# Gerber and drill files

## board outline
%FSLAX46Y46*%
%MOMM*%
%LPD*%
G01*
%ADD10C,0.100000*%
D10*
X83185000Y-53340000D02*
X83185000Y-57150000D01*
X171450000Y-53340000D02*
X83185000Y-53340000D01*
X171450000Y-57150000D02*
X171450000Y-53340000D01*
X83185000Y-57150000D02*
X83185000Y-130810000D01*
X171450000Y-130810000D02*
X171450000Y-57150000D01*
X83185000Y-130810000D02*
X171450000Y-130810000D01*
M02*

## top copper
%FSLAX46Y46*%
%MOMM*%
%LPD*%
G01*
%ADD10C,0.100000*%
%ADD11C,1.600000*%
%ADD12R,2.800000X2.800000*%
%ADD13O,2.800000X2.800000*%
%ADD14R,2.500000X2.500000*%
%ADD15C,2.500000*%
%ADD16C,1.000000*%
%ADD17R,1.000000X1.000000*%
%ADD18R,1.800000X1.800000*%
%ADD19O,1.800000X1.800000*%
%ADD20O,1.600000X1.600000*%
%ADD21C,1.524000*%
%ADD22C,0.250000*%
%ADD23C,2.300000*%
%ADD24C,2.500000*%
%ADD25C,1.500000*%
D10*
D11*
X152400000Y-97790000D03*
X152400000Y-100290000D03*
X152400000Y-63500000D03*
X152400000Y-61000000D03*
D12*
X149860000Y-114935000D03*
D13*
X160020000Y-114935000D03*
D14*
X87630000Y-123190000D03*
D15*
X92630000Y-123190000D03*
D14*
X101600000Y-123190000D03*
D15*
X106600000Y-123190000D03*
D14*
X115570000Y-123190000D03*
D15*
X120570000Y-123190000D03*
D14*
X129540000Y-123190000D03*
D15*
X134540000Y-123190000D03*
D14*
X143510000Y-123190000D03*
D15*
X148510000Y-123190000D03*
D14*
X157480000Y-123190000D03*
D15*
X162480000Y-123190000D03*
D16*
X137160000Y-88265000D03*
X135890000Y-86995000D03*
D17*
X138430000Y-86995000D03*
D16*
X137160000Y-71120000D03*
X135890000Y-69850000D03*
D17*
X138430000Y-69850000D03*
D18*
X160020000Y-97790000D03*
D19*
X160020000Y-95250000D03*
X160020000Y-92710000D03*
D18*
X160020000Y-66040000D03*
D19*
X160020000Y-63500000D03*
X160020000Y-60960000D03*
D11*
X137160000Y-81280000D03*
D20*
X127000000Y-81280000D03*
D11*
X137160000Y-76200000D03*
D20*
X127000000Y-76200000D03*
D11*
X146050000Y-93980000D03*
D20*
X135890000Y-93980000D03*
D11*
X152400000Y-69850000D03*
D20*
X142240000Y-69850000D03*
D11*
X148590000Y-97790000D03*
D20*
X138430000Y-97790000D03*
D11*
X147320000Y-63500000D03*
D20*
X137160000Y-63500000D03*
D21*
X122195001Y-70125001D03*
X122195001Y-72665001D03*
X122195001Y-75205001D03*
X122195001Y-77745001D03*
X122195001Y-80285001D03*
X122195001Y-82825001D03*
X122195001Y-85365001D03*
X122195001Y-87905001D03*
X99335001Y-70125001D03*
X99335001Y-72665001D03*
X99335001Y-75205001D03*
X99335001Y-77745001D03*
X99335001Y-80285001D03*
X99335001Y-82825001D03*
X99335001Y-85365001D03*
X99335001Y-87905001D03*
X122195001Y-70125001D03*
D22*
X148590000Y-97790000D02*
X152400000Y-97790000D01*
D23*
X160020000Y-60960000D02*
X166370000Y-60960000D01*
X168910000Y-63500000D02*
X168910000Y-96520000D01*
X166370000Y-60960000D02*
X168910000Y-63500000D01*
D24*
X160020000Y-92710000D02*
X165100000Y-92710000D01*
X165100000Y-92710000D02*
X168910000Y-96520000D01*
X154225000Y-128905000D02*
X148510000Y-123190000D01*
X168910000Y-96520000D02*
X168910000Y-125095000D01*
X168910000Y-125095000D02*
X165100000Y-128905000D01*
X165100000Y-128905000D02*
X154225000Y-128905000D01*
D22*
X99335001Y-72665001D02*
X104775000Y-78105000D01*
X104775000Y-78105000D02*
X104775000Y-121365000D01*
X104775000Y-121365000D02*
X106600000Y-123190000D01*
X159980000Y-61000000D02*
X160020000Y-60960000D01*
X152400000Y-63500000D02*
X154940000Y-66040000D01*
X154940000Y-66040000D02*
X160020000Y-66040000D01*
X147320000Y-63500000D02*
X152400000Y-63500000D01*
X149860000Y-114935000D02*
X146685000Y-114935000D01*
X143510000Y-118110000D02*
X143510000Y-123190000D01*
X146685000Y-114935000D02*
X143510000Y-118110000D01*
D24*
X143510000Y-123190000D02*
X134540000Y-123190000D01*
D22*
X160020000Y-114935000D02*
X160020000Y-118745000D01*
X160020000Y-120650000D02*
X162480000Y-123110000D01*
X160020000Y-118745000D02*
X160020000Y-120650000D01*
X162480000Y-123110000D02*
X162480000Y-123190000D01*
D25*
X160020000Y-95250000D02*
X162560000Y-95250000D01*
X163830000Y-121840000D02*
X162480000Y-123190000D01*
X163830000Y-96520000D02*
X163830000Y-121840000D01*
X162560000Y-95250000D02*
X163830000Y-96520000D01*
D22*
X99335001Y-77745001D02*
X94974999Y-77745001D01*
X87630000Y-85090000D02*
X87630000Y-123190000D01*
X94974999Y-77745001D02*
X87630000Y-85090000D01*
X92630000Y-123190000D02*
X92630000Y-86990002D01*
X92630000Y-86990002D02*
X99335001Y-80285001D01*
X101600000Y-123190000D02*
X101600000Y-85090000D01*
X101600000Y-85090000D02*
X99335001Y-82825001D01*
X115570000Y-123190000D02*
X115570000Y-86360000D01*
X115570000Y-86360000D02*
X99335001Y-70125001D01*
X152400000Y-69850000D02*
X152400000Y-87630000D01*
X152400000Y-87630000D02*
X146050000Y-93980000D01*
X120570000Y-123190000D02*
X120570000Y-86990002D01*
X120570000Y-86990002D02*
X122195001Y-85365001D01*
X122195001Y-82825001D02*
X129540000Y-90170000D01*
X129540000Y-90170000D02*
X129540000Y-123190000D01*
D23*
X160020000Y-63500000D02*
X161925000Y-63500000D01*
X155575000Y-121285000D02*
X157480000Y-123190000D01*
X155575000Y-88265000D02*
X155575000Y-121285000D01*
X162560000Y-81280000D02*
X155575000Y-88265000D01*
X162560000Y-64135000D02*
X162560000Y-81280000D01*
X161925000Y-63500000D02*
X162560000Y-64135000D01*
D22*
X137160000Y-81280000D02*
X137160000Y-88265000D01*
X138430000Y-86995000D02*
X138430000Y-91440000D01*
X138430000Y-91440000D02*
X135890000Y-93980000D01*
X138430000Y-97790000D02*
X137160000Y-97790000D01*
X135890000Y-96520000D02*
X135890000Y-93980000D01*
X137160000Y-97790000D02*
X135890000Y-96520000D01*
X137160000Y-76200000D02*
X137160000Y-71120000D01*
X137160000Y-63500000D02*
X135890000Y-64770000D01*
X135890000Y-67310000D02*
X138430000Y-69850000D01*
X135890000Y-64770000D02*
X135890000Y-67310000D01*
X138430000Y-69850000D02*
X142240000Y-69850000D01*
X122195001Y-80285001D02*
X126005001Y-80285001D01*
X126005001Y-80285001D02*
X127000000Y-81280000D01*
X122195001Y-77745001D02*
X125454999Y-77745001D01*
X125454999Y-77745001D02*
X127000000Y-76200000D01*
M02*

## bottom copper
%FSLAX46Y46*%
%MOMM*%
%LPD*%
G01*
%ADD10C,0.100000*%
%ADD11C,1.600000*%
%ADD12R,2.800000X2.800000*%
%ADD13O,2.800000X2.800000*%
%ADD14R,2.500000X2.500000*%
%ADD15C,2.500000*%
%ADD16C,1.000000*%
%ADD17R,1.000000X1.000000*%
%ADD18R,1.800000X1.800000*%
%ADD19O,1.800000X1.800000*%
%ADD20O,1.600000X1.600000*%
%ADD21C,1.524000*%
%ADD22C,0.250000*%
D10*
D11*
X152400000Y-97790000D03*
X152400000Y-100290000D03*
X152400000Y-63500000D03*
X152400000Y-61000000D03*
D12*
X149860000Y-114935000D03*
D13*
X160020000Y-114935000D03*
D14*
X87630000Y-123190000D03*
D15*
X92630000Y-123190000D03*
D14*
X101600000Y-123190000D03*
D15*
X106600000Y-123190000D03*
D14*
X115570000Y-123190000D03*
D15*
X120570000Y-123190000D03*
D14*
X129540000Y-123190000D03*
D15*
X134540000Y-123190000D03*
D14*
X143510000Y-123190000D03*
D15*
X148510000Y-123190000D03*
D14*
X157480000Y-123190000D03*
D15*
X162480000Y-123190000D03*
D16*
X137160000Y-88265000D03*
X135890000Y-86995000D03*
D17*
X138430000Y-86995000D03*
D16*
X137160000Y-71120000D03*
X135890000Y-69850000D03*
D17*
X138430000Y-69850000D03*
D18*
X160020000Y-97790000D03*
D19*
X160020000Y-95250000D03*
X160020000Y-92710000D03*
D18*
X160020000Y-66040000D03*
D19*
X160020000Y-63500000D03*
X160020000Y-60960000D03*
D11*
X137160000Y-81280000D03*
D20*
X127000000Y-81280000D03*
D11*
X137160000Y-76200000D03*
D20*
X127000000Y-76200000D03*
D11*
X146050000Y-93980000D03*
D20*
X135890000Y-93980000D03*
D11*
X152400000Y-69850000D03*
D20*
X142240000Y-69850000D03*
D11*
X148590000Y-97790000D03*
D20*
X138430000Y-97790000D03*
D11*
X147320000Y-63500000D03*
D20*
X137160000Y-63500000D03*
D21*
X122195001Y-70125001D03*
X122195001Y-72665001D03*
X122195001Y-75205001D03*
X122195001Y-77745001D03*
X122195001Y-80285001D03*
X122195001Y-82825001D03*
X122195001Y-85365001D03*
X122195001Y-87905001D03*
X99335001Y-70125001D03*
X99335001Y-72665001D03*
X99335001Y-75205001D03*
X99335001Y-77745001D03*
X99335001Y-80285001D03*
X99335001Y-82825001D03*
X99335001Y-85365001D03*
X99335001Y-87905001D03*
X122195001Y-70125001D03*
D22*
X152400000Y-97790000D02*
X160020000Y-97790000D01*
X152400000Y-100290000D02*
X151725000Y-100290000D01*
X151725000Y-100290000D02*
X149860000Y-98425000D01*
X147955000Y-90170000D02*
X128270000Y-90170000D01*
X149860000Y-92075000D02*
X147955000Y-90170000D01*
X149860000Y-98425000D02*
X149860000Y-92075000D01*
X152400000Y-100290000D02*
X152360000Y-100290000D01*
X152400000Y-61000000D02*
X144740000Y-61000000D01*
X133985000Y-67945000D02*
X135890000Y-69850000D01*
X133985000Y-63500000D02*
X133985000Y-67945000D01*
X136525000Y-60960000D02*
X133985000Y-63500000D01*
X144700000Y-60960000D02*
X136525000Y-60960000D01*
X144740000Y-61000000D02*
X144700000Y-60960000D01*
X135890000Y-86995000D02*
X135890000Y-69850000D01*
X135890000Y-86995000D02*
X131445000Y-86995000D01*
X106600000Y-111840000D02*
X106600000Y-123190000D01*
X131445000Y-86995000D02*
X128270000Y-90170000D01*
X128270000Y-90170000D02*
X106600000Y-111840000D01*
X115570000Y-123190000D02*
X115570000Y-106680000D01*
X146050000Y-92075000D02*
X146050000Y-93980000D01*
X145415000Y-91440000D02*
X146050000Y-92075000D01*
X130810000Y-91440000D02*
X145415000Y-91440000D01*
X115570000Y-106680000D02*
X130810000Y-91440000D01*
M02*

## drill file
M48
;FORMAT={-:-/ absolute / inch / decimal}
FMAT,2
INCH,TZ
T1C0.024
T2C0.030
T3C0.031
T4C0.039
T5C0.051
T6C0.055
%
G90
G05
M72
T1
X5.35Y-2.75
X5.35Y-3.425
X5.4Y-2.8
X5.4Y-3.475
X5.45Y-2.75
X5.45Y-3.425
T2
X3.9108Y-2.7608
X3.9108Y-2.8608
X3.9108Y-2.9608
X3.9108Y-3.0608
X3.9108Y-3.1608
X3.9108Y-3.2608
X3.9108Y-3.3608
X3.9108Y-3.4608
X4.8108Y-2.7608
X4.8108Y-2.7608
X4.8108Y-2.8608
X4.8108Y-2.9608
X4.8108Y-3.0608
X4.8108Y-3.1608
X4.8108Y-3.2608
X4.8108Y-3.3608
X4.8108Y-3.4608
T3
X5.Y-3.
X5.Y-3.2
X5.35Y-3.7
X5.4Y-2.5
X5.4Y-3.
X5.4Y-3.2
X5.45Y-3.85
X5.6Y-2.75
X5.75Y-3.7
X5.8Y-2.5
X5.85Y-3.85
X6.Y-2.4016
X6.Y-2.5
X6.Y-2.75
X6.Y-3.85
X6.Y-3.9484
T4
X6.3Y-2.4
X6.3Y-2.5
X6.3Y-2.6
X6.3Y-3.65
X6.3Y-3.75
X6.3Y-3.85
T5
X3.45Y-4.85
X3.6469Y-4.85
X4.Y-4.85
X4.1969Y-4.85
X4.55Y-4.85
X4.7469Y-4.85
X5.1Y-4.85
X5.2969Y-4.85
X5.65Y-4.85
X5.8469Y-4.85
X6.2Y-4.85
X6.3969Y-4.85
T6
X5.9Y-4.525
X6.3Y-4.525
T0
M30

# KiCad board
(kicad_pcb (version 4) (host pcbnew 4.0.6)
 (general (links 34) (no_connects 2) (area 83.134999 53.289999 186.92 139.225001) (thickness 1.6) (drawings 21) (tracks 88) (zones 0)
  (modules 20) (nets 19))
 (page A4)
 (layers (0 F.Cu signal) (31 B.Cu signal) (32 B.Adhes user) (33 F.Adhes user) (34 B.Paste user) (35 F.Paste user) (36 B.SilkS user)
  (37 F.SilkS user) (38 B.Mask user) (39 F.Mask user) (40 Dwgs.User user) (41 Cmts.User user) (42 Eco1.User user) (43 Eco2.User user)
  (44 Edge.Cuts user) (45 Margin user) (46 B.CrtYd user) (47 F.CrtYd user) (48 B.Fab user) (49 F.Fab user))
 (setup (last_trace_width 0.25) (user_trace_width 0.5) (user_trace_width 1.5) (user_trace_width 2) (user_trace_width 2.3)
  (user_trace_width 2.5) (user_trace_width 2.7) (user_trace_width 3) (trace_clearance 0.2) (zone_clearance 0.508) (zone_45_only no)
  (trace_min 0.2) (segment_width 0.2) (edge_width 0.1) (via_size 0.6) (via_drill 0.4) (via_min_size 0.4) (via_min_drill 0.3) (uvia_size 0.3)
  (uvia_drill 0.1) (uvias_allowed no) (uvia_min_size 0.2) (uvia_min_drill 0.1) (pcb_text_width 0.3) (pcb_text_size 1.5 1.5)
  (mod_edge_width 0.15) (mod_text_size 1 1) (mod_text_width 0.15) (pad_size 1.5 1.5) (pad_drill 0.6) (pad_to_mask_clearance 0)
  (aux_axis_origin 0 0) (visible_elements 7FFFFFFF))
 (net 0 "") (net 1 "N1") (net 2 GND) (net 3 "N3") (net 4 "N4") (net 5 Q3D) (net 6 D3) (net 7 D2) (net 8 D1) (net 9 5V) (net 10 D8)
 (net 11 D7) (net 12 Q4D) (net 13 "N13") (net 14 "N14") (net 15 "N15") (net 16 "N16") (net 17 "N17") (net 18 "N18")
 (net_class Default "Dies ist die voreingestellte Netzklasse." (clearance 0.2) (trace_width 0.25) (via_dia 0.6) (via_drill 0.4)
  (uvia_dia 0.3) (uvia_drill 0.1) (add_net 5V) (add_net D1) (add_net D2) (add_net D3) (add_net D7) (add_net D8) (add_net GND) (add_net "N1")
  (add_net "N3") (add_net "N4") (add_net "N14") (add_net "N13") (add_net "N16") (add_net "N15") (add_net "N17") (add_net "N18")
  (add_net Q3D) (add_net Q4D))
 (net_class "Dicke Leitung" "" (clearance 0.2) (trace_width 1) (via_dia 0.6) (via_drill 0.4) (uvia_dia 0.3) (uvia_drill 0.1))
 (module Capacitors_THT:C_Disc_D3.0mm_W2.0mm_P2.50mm (layer F.Cu) (at 152.4 97.79 270)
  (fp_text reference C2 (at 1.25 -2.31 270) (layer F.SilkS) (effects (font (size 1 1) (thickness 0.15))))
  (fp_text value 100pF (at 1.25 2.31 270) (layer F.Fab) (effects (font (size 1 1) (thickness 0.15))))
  (pad 1 thru_hole circle (at 0 0 270) (size 1.6 1.6) (drill 0.8) (layers *.Cu *.Mask) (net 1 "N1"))
  (pad 2 thru_hole circle (at 2.5 0 270) (size 1.6 1.6) (drill 0.8) (layers *.Cu *.Mask) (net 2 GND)))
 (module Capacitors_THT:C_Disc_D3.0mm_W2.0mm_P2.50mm (layer F.Cu) (at 152.4 63.5 90)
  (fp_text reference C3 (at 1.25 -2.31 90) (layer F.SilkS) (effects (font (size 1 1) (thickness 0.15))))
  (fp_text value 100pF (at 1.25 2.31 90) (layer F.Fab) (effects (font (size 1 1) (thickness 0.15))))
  (pad 1 thru_hole circle (at 0 0 90) (size 1.6 1.6) (drill 0.8) (layers *.Cu *.Mask) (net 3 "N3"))
  (pad 2 thru_hole circle (at 2.5 0 90) (size 1.6 1.6) (drill 0.8) (layers *.Cu *.Mask) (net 2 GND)))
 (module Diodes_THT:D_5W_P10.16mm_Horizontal (layer F.Cu) (at 149.86 114.935)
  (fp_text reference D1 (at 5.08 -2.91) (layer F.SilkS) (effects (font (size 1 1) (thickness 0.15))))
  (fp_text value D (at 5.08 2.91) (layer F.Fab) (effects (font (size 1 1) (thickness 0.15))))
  (pad 1 thru_hole rect (at 0 0) (size 2.8 2.8) (drill 1.4) (layers *.Cu *.Mask) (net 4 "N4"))
  (pad 2 thru_hole oval (at 10.16 0) (size 2.8 2.8) (drill 1.4) (layers *.Cu *.Mask) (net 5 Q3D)))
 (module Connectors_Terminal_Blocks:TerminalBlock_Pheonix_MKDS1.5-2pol (layer F.Cu) (at 87.63 123.19)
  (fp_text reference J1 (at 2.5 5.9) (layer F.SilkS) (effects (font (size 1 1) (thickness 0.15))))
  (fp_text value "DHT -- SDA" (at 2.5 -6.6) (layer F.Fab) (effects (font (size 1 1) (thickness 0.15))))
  (pad 1 thru_hole rect (at 0 0) (size 2.5 2.5) (drill 1.3) (layers *.Cu *.Mask) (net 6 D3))
  (pad 2 thru_hole circle (at 5 0) (size 2.5 2.5) (drill 1.3) (layers *.Cu *.Mask) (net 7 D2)))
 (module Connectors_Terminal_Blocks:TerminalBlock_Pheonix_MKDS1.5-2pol (layer F.Cu) (at 101.6 123.19)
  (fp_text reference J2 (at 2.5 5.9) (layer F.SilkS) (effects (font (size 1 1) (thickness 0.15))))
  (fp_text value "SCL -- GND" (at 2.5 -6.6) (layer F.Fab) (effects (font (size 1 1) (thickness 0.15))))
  (pad 1 thru_hole rect (at 0 0) (size 2.5 2.5) (drill 1.3) (layers *.Cu *.Mask) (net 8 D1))
  (pad 2 thru_hole circle (at 5 0) (size 2.5 2.5) (drill 1.3) (layers *.Cu *.Mask) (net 2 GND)))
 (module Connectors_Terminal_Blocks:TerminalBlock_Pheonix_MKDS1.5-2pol (layer F.Cu) (at 115.57 123.19)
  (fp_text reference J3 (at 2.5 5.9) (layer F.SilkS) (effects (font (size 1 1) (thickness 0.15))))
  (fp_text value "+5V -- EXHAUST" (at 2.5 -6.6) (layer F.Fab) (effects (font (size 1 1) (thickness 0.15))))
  (pad 1 thru_hole rect (at 0 0) (size 2.5 2.5) (drill 1.3) (layers *.Cu *.Mask) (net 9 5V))
  (pad 2 thru_hole circle (at 5 0) (size 2.5 2.5) (drill 1.3) (layers *.Cu *.Mask) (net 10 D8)))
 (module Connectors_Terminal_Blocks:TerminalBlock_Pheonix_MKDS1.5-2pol (layer F.Cu) (at 129.54 123.19)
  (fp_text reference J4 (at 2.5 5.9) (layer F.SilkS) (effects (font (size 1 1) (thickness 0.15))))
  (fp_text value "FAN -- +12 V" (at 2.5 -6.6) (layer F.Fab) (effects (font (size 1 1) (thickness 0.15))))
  (pad 1 thru_hole rect (at 0 0) (size 2.5 2.5) (drill 1.3) (layers *.Cu *.Mask) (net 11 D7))
  (pad 2 thru_hole circle (at 5 0) (size 2.5 2.5) (drill 1.3) (layers *.Cu *.Mask) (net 4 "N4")))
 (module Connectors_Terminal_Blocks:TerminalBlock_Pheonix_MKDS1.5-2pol (layer F.Cu) (at 143.51 123.19)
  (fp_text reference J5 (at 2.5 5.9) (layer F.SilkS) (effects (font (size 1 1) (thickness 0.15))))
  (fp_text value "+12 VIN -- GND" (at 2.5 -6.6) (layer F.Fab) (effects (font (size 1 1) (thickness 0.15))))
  (pad 1 thru_hole rect (at 0 0) (size 2.5 2.5) (drill 1.3) (layers *.Cu *.Mask) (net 4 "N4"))
  (pad 2 thru_hole circle (at 5 0) (size 2.5 2.5) (drill 1.3) (layers *.Cu *.Mask) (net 2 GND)))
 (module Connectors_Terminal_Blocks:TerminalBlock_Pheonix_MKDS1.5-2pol (layer F.Cu) (at 157.48 123.19)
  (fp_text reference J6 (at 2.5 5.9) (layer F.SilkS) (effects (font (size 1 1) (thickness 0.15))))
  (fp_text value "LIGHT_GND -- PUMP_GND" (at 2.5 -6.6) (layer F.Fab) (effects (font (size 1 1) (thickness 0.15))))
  (pad 1 thru_hole rect (at 0 0) (size 2.5 2.5) (drill 1.3) (layers *.Cu *.Mask) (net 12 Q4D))
  (pad 2 thru_hole circle (at 5 0) (size 2.5 2.5) (drill 1.3) (layers *.Cu *.Mask) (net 5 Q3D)))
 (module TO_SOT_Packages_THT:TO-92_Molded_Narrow (layer F.Cu) (at 138.43 86.995 180)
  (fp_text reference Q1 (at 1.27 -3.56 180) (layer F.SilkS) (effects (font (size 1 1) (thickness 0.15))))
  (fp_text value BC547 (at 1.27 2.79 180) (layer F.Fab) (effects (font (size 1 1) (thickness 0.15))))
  (pad 2 thru_hole circle (at 1.27 -1.27 270) (size 1 1) (drill 0.6) (layers *.Cu *.Mask) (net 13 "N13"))
  (pad 3 thru_hole circle (at 2.54 0 270) (size 1 1) (drill 0.6) (layers *.Cu *.Mask) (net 2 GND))
  (pad 1 thru_hole rect (at 0 0 270) (size 1 1) (drill 0.6) (layers *.Cu *.Mask) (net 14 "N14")))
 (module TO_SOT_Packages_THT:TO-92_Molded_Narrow (layer F.Cu) (at 138.43 69.85 180)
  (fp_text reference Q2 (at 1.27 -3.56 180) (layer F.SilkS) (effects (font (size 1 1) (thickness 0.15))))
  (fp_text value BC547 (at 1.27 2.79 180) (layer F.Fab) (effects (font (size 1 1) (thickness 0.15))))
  (pad 2 thru_hole circle (at 1.27 -1.27 270) (size 1 1) (drill 0.6) (layers *.Cu *.Mask) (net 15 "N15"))
  (pad 3 thru_hole circle (at 2.54 0 270) (size 1 1) (drill 0.6) (layers *.Cu *.Mask) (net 2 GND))
  (pad 1 thru_hole rect (at 0 0 270) (size 1 1) (drill 0.6) (layers *.Cu *.Mask) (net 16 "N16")))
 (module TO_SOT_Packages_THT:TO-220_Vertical (layer F.Cu) (at 160.02 97.79 90)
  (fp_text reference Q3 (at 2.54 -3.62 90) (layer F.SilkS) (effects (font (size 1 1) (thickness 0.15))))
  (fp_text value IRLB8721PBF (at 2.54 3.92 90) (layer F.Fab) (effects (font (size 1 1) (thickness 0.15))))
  (pad 1 thru_hole rect (at 0 0 90) (size 1.8 1.8) (drill 1) (layers *.Cu *.Mask) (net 1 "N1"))
  (pad 2 thru_hole oval (at 2.54 0 90) (size 1.8 1.8) (drill 1) (layers *.Cu *.Mask) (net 5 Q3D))
  (pad 3 thru_hole oval (at 5.08 0 90) (size 1.8 1.8) (drill 1) (layers *.Cu *.Mask) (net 2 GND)))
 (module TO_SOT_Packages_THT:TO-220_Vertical (layer F.Cu) (at 160.02 66.04 90)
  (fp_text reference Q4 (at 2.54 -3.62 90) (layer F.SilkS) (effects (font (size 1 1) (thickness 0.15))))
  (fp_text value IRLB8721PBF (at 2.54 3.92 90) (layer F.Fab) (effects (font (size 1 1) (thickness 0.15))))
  (pad 1 thru_hole rect (at 0 0 90) (size 1.8 1.8) (drill 1) (layers *.Cu *.Mask) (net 3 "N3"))
  (pad 2 thru_hole oval (at 2.54 0 90) (size 1.8 1.8) (drill 1) (layers *.Cu *.Mask) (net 12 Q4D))
  (pad 3 thru_hole oval (at 5.08 0 90) (size 1.8 1.8) (drill 1) (layers *.Cu *.Mask) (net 2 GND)))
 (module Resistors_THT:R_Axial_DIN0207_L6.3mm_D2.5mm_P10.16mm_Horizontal (layer F.Cu) (at 137.16 81.28 180)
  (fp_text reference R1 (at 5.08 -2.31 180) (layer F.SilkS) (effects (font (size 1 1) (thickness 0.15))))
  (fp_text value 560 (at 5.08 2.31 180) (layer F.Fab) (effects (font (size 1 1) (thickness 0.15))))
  (pad 1 thru_hole circle (at 0 0 180) (size 1.6 1.6) (drill 0.8) (layers *.Cu *.Mask) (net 13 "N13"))
  (pad 2 thru_hole oval (at 10.16 0 180) (size 1.6 1.6) (drill 0.8) (layers *.Cu *.Mask) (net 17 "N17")))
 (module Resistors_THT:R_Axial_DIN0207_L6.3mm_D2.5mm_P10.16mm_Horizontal (layer F.Cu) (at 137.16 76.2 180)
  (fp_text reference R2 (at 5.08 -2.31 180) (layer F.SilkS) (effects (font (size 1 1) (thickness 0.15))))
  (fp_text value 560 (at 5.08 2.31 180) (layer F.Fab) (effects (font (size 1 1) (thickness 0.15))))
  (pad 1 thru_hole circle (at 0 0 180) (size 1.6 1.6) (drill 0.8) (layers *.Cu *.Mask) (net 15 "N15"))
  (pad 2 thru_hole oval (at 10.16 0 180) (size 1.6 1.6) (drill 0.8) (layers *.Cu *.Mask) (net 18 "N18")))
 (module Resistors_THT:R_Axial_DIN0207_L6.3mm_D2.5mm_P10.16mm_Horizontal (layer F.Cu) (at 146.05 93.98 180)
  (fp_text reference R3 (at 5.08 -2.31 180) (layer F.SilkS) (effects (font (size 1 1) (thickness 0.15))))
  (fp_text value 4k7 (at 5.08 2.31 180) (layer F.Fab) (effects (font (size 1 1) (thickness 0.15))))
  (pad 1 thru_hole circle (at 0 0 180) (size 1.6 1.6) (drill 0.8) (layers *.Cu *.Mask) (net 9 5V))
  (pad 2 thru_hole oval (at 10.16 0 180) (size 1.6 1.6) (drill 0.8) (layers *.Cu *.Mask) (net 14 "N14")))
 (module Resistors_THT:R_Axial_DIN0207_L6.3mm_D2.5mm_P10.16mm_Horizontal (layer F.Cu) (at 152.4 69.85 180)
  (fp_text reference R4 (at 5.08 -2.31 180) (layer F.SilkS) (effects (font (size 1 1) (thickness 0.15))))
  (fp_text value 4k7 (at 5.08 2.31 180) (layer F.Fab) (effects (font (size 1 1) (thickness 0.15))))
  (pad 1 thru_hole circle (at 0 0 180) (size 1.6 1.6) (drill 0.8) (layers *.Cu *.Mask) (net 9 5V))
  (pad 2 thru_hole oval (at 10.16 0 180) (size 1.6 1.6) (drill 0.8) (layers *.Cu *.Mask) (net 16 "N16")))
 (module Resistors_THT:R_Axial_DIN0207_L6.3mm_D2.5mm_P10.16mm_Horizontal (layer F.Cu) (at 148.59 97.79 180)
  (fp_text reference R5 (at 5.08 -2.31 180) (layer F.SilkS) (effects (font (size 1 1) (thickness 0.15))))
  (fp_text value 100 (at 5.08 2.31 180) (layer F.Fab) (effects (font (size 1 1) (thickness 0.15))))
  (pad 1 thru_hole circle (at 0 0 180) (size 1.6 1.6) (drill 0.8) (layers *.Cu *.Mask) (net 1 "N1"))
  (pad 2 thru_hole oval (at 10.16 0 180) (size 1.6 1.6) (drill 0.8) (layers *.Cu *.Mask) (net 14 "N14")))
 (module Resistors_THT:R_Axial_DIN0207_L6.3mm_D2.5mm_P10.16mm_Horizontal (layer F.Cu) (at 147.32 63.5 180)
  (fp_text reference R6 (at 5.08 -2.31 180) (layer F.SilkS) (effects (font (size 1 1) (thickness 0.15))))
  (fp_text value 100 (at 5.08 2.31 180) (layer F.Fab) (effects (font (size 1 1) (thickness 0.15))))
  (pad 1 thru_hole circle (at 0 0 180) (size 1.6 1.6) (drill 0.8) (layers *.Cu *.Mask) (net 3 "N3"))
  (pad 2 thru_hole oval (at 10.16 0 180) (size 1.6 1.6) (drill 0.8) (layers *.Cu *.Mask) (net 16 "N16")))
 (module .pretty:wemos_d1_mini (layer F.Cu) (at 110.765001 79.015001)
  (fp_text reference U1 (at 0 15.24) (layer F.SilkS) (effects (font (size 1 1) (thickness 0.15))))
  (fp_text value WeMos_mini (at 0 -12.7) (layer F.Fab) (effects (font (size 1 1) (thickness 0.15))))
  (pad 5 thru_hole circle (at 11.43 -8.89) (size 1.524 1.524) (drill 0.762) (layers *.Cu *.Mask) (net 7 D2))
  (pad 10 thru_hole circle (at 11.43 -6.35) (size 1.524 1.524) (drill 0.762) (layers *.Cu *.Mask))
  (pad 11 thru_hole circle (at 11.43 -3.81) (size 1.524 1.524) (drill 0.762) (layers *.Cu *.Mask))
  (pad 12 thru_hole circle (at 11.43 -1.27) (size 1.524 1.524) (drill 0.762) (layers *.Cu *.Mask) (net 18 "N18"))
  (pad 13 thru_hole circle (at 11.43 1.27) (size 1.524 1.524) (drill 0.762) (layers *.Cu *.Mask) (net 17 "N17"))
  (pad 14 thru_hole circle (at 11.43 3.81) (size 1.524 1.524) (drill 0.762) (layers *.Cu *.Mask) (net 11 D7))
  (pad 15 thru_hole circle (at 11.43 6.35) (size 1.524 1.524) (drill 0.762) (layers *.Cu *.Mask) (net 10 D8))
  (pad 16 thru_hole circle (at 11.43 8.89) (size 1.524 1.524) (drill 0.762) (layers *.Cu *.Mask))
  (pad 1 thru_hole circle (at -11.43 -8.89) (size 1.524 1.524) (drill 0.762) (layers *.Cu *.Mask) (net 9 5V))
  (pad 2 thru_hole circle (at -11.43 -6.35) (size 1.524 1.524) (drill 0.762) (layers *.Cu *.Mask) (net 2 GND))
  (pad 3 thru_hole circle (at -11.43 -3.81) (size 1.524 1.524) (drill 0.762) (layers *.Cu *.Mask))
  (pad 4 thru_hole circle (at -11.43 -1.27) (size 1.524 1.524) (drill 0.762) (layers *.Cu *.Mask) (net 6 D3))
  (pad 5 thru_hole circle (at -11.43 1.27) (size 1.524 1.524) (drill 0.762) (layers *.Cu *.Mask) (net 7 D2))
  (pad 6 thru_hole circle (at -11.43 3.81) (size 1.524 1.524) (drill 0.762) (layers *.Cu *.Mask) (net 8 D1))
  (pad 7 thru_hole circle (at -11.43 6.35) (size 1.524 1.524) (drill 0.762) (layers *.Cu *.Mask))
  (pad 8 thru_hole circle (at -11.43 8.89) (size 1.524 1.524) (drill 0.762) (layers *.Cu *.Mask))
  (pad 9 thru_hole circle (at 11.43 -8.89) (size 1.524 1.524) (drill 0.762) (layers *.Cu *.Mask)))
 (gr_line (start 83.185 53.34) (end 83.185 57.15) (angle 90) (layer Edge.Cuts) (width 0.1))
 (gr_line (start 171.45 53.34) (end 83.185 53.34) (angle 90) (layer Edge.Cuts) (width 0.1))
 (gr_line (start 171.45 57.15) (end 171.45 53.34) (angle 90) (layer Edge.Cuts) (width 0.1))
 (gr_line (start 83.185 57.15) (end 83.185 130.81) (angle 90) (layer Edge.Cuts) (width 0.1))
 (gr_line (start 171.45 130.81) (end 171.45 57.15) (angle 90) (layer Edge.Cuts) (width 0.1))
 (gr_line (start 83.185 130.81) (end 171.45 130.81) (angle 90) (layer Edge.Cuts) (width 0.1))
 (segment (start 152.4 97.79) (end 160.02 97.79) (width 0.25) (layer B.Cu) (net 1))
 (segment (start 148.59 97.79) (end 152.4 97.79) (width 0.25) (layer F.Cu) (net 1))
 (segment (start 152.4 100.29) (end 151.725 100.29) (width 0.25) (layer B.Cu) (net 2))
 (segment (start 151.725 100.29) (end 149.86 98.425) (width 0.25) (layer B.Cu) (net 2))
 (segment (start 147.955 90.17) (end 128.27 90.17) (width 0.25) (layer B.Cu) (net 2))
 (segment (start 149.86 92.075) (end 147.955 90.17) (width 0.25) (layer B.Cu) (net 2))
 (segment (start 149.86 98.425) (end 149.86 92.075) (width 0.25) (layer B.Cu) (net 2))
 (segment (start 152.4 100.29) (end 152.36 100.29) (width 0.25) (layer B.Cu) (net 2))
 (segment (start 152.4 61) (end 144.74 61) (width 0.25) (layer B.Cu) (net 2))
 (segment (start 133.985 67.945) (end 135.89 69.85) (width 0.25) (layer B.Cu) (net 2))
 (segment (start 133.985 63.5) (end 133.985 67.945) (width 0.25) (layer B.Cu) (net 2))
 (segment (start 136.525 60.96) (end 133.985 63.5) (width 0.25) (layer B.Cu) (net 2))
 (segment (start 144.7 60.96) (end 136.525 60.96) (width 0.25) (layer B.Cu) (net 2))
 (segment (start 144.74 61) (end 144.7 60.96) (width 0.25) (layer B.Cu) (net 2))
 (segment (start 135.89 86.995) (end 135.89 69.85) (width 0.25) (layer B.Cu) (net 2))
 (segment (start 135.89 86.995) (end 131.445 86.995) (width 0.25) (layer B.Cu) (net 2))
 (segment (start 106.6 111.84) (end 106.6 123.19) (width 0.25) (layer B.Cu) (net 2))
 (segment (start 131.445 86.995) (end 128.27 90.17) (width 0.25) (layer B.Cu) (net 2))
 (segment (start 128.27 90.17) (end 106.6 111.84) (width 0.25) (layer B.Cu) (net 2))
 (segment (start 160.02 60.96) (end 166.37 60.96) (width 2.3) (layer F.Cu) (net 2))
 (segment (start 168.91 63.5) (end 168.91 96.52) (width 2.3) (layer F.Cu) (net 2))
 (segment (start 166.37 60.96) (end 168.91 63.5) (width 2.3) (layer F.Cu) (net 2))
 (segment (start 160.02 92.71) (end 165.1 92.71) (width 2.5) (layer F.Cu) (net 2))
 (segment (start 165.1 92.71) (end 168.91 96.52) (width 2.5) (layer F.Cu) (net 2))
 (segment (start 154.225 128.905) (end 148.51 123.19) (width 2.5) (layer F.Cu) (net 2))
 (segment (start 168.91 96.52) (end 168.91 125.095) (width 2.5) (layer F.Cu) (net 2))
 (segment (start 168.91 125.095) (end 165.1 128.905) (width 2.5) (layer F.Cu) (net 2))
 (segment (start 165.1 128.905) (end 154.225 128.905) (width 2.5) (layer F.Cu) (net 2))
 (segment (start 99.335001 72.665001) (end 104.775 78.105) (width 0.25) (layer F.Cu) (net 2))
 (segment (start 104.775 78.105) (end 104.775 121.365) (width 0.25) (layer F.Cu) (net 2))
 (segment (start 104.775 121.365) (end 106.6 123.19) (width 0.25) (layer F.Cu) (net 2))
 (segment (start 159.98 61) (end 160.02 60.96) (width 0.25) (layer F.Cu) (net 2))
 (segment (start 152.4 63.5) (end 154.94 66.04) (width 0.25) (layer F.Cu) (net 3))
 (segment (start 154.94 66.04) (end 160.02 66.04) (width 0.25) (layer F.Cu) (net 3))
 (segment (start 147.32 63.5) (end 152.4 63.5) (width 0.25) (layer F.Cu) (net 3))
 (segment (start 149.86 114.935) (end 146.685 114.935) (width 0.25) (layer F.Cu) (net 4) (status 400000))
 (segment (start 143.51 118.11) (end 143.51 123.19) (width 0.25) (layer F.Cu) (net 4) (status 800000))
 (segment (start 146.685 114.935) (end 143.51 118.11) (width 0.25) (layer F.Cu) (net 4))
 (segment (start 143.51 123.19) (end 134.54 123.19) (width 2.5) (layer F.Cu) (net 4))
 (segment (start 160.02 114.935) (end 160.02 118.745) (width 0.25) (layer F.Cu) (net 5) (status 400000))
 (segment (start 160.02 120.65) (end 162.48 123.11) (width 0.25) (layer F.Cu) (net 5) (status 800000))
 (segment (start 160.02 118.745) (end 160.02 120.65) (width 0.25) (layer F.Cu) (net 5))
 (segment (start 162.48 123.11) (end 162.48 123.19) (width 0.25) (layer F.Cu) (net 5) (status C00000))
 (segment (start 160.02 95.25) (end 162.56 95.25) (width 1.5) (layer F.Cu) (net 5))
 (segment (start 163.83 121.84) (end 162.48 123.19) (width 1.5) (layer F.Cu) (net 5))
 (segment (start 163.83 96.52) (end 163.83 121.84) (width 1.5) (layer F.Cu) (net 5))
 (segment (start 162.56 95.25) (end 163.83 96.52) (width 1.5) (layer F.Cu) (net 5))
 (segment (start 99.335001 77.745001) (end 94.974999 77.745001) (width 0.25) (layer F.Cu) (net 6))
 (segment (start 87.63 85.09) (end 87.63 123.19) (width 0.25) (layer F.Cu) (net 6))
 (segment (start 94.974999 77.745001) (end 87.63 85.09) (width 0.25) (layer F.Cu) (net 6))
 (segment (start 92.63 123.19) (end 92.63 86.990002) (width 0.25) (layer F.Cu) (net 7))
 (segment (start 92.63 86.990002) (end 99.335001 80.285001) (width 0.25) (layer F.Cu) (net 7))
 (segment (start 101.6 123.19) (end 101.6 85.09) (width 0.25) (layer F.Cu) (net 8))
 (segment (start 101.6 85.09) (end 99.335001 82.825001) (width 0.25) (layer F.Cu) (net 8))
 (segment (start 115.57 123.19) (end 115.57 106.68) (width 0.25) (layer B.Cu) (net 9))
 (segment (start 146.05 92.075) (end 146.05 93.98) (width 0.25) (layer B.Cu) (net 9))
 (segment (start 145.415 91.44) (end 146.05 92.075) (width 0.25) (layer B.Cu) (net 9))
 (segment (start 130.81 91.44) (end 145.415 91.44) (width 0.25) (layer B.Cu) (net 9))
 (segment (start 115.57 106.68) (end 130.81 91.44) (width 0.25) (layer B.Cu) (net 9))
 (segment (start 115.57 123.19) (end 115.57 86.36) (width 0.25) (layer F.Cu) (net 9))
 (segment (start 115.57 86.36) (end 99.335001 70.125001) (width 0.25) (layer F.Cu) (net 9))
 (segment (start 152.4 69.85) (end 152.4 87.63) (width 0.25) (layer F.Cu) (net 9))
 (segment (start 152.4 87.63) (end 146.05 93.98) (width 0.25) (layer F.Cu) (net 9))
 (segment (start 120.57 123.19) (end 120.57 86.990002) (width 0.25) (layer F.Cu) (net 10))
 (segment (start 120.57 86.990002) (end 122.195001 85.365001) (width 0.25) (layer F.Cu) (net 10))
 (segment (start 122.195001 82.825001) (end 129.54 90.17) (width 0.25) (layer F.Cu) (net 11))
 (segment (start 129.54 90.17) (end 129.54 123.19) (width 0.25) (layer F.Cu) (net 11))
 (segment (start 160.02 63.5) (end 161.925 63.5) (width 2.3) (layer F.Cu) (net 12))
 (segment (start 155.575 121.285) (end 157.48 123.19) (width 2.3) (layer F.Cu) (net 12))
 (segment (start 155.575 88.265) (end 155.575 121.285) (width 2.3) (layer F.Cu) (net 12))
 (segment (start 162.56 81.28) (end 155.575 88.265) (width 2.3) (layer F.Cu) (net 12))
 (segment (start 162.56 64.135) (end 162.56 81.28) (width 2.3) (layer F.Cu) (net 12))
 (segment (start 161.925 63.5) (end 162.56 64.135) (width 2.3) (layer F.Cu) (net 12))
 (segment (start 137.16 81.28) (end 137.16 88.265) (width 0.25) (layer F.Cu) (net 13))
 (segment (start 138.43 86.995) (end 138.43 91.44) (width 0.25) (layer F.Cu) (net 14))
 (segment (start 138.43 91.44) (end 135.89 93.98) (width 0.25) (layer F.Cu) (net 14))
 (segment (start 138.43 97.79) (end 137.16 97.79) (width 0.25) (layer F.Cu) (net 14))
 (segment (start 135.89 96.52) (end 135.89 93.98) (width 0.25) (layer F.Cu) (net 14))
 (segment (start 137.16 97.79) (end 135.89 96.52) (width 0.25) (layer F.Cu) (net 14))
 (segment (start 137.16 76.2) (end 137.16 71.12) (width 0.25) (layer F.Cu) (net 15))
 (segment (start 137.16 63.5) (end 135.89 64.77) (width 0.25) (layer F.Cu) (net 16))
 (segment (start 135.89 67.31) (end 138.43 69.85) (width 0.25) (layer F.Cu) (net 16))
 (segment (start 135.89 64.77) (end 135.89 67.31) (width 0.25) (layer F.Cu) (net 16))
 (segment (start 138.43 69.85) (end 142.24 69.85) (width 0.25) (layer F.Cu) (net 16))
 (segment (start 122.195001 80.285001) (end 126.005001 80.285001) (width 0.25) (layer F.Cu) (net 17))
 (segment (start 126.005001 80.285001) (end 127 81.28) (width 0.25) (layer F.Cu) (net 17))
 (segment (start 122.195001 77.745001) (end 125.454999 77.745001) (width 0.25) (layer F.Cu) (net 18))
 (segment (start 125.454999 77.745001) (end 127 76.2) (width 0.25) (layer F.Cu) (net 18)))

